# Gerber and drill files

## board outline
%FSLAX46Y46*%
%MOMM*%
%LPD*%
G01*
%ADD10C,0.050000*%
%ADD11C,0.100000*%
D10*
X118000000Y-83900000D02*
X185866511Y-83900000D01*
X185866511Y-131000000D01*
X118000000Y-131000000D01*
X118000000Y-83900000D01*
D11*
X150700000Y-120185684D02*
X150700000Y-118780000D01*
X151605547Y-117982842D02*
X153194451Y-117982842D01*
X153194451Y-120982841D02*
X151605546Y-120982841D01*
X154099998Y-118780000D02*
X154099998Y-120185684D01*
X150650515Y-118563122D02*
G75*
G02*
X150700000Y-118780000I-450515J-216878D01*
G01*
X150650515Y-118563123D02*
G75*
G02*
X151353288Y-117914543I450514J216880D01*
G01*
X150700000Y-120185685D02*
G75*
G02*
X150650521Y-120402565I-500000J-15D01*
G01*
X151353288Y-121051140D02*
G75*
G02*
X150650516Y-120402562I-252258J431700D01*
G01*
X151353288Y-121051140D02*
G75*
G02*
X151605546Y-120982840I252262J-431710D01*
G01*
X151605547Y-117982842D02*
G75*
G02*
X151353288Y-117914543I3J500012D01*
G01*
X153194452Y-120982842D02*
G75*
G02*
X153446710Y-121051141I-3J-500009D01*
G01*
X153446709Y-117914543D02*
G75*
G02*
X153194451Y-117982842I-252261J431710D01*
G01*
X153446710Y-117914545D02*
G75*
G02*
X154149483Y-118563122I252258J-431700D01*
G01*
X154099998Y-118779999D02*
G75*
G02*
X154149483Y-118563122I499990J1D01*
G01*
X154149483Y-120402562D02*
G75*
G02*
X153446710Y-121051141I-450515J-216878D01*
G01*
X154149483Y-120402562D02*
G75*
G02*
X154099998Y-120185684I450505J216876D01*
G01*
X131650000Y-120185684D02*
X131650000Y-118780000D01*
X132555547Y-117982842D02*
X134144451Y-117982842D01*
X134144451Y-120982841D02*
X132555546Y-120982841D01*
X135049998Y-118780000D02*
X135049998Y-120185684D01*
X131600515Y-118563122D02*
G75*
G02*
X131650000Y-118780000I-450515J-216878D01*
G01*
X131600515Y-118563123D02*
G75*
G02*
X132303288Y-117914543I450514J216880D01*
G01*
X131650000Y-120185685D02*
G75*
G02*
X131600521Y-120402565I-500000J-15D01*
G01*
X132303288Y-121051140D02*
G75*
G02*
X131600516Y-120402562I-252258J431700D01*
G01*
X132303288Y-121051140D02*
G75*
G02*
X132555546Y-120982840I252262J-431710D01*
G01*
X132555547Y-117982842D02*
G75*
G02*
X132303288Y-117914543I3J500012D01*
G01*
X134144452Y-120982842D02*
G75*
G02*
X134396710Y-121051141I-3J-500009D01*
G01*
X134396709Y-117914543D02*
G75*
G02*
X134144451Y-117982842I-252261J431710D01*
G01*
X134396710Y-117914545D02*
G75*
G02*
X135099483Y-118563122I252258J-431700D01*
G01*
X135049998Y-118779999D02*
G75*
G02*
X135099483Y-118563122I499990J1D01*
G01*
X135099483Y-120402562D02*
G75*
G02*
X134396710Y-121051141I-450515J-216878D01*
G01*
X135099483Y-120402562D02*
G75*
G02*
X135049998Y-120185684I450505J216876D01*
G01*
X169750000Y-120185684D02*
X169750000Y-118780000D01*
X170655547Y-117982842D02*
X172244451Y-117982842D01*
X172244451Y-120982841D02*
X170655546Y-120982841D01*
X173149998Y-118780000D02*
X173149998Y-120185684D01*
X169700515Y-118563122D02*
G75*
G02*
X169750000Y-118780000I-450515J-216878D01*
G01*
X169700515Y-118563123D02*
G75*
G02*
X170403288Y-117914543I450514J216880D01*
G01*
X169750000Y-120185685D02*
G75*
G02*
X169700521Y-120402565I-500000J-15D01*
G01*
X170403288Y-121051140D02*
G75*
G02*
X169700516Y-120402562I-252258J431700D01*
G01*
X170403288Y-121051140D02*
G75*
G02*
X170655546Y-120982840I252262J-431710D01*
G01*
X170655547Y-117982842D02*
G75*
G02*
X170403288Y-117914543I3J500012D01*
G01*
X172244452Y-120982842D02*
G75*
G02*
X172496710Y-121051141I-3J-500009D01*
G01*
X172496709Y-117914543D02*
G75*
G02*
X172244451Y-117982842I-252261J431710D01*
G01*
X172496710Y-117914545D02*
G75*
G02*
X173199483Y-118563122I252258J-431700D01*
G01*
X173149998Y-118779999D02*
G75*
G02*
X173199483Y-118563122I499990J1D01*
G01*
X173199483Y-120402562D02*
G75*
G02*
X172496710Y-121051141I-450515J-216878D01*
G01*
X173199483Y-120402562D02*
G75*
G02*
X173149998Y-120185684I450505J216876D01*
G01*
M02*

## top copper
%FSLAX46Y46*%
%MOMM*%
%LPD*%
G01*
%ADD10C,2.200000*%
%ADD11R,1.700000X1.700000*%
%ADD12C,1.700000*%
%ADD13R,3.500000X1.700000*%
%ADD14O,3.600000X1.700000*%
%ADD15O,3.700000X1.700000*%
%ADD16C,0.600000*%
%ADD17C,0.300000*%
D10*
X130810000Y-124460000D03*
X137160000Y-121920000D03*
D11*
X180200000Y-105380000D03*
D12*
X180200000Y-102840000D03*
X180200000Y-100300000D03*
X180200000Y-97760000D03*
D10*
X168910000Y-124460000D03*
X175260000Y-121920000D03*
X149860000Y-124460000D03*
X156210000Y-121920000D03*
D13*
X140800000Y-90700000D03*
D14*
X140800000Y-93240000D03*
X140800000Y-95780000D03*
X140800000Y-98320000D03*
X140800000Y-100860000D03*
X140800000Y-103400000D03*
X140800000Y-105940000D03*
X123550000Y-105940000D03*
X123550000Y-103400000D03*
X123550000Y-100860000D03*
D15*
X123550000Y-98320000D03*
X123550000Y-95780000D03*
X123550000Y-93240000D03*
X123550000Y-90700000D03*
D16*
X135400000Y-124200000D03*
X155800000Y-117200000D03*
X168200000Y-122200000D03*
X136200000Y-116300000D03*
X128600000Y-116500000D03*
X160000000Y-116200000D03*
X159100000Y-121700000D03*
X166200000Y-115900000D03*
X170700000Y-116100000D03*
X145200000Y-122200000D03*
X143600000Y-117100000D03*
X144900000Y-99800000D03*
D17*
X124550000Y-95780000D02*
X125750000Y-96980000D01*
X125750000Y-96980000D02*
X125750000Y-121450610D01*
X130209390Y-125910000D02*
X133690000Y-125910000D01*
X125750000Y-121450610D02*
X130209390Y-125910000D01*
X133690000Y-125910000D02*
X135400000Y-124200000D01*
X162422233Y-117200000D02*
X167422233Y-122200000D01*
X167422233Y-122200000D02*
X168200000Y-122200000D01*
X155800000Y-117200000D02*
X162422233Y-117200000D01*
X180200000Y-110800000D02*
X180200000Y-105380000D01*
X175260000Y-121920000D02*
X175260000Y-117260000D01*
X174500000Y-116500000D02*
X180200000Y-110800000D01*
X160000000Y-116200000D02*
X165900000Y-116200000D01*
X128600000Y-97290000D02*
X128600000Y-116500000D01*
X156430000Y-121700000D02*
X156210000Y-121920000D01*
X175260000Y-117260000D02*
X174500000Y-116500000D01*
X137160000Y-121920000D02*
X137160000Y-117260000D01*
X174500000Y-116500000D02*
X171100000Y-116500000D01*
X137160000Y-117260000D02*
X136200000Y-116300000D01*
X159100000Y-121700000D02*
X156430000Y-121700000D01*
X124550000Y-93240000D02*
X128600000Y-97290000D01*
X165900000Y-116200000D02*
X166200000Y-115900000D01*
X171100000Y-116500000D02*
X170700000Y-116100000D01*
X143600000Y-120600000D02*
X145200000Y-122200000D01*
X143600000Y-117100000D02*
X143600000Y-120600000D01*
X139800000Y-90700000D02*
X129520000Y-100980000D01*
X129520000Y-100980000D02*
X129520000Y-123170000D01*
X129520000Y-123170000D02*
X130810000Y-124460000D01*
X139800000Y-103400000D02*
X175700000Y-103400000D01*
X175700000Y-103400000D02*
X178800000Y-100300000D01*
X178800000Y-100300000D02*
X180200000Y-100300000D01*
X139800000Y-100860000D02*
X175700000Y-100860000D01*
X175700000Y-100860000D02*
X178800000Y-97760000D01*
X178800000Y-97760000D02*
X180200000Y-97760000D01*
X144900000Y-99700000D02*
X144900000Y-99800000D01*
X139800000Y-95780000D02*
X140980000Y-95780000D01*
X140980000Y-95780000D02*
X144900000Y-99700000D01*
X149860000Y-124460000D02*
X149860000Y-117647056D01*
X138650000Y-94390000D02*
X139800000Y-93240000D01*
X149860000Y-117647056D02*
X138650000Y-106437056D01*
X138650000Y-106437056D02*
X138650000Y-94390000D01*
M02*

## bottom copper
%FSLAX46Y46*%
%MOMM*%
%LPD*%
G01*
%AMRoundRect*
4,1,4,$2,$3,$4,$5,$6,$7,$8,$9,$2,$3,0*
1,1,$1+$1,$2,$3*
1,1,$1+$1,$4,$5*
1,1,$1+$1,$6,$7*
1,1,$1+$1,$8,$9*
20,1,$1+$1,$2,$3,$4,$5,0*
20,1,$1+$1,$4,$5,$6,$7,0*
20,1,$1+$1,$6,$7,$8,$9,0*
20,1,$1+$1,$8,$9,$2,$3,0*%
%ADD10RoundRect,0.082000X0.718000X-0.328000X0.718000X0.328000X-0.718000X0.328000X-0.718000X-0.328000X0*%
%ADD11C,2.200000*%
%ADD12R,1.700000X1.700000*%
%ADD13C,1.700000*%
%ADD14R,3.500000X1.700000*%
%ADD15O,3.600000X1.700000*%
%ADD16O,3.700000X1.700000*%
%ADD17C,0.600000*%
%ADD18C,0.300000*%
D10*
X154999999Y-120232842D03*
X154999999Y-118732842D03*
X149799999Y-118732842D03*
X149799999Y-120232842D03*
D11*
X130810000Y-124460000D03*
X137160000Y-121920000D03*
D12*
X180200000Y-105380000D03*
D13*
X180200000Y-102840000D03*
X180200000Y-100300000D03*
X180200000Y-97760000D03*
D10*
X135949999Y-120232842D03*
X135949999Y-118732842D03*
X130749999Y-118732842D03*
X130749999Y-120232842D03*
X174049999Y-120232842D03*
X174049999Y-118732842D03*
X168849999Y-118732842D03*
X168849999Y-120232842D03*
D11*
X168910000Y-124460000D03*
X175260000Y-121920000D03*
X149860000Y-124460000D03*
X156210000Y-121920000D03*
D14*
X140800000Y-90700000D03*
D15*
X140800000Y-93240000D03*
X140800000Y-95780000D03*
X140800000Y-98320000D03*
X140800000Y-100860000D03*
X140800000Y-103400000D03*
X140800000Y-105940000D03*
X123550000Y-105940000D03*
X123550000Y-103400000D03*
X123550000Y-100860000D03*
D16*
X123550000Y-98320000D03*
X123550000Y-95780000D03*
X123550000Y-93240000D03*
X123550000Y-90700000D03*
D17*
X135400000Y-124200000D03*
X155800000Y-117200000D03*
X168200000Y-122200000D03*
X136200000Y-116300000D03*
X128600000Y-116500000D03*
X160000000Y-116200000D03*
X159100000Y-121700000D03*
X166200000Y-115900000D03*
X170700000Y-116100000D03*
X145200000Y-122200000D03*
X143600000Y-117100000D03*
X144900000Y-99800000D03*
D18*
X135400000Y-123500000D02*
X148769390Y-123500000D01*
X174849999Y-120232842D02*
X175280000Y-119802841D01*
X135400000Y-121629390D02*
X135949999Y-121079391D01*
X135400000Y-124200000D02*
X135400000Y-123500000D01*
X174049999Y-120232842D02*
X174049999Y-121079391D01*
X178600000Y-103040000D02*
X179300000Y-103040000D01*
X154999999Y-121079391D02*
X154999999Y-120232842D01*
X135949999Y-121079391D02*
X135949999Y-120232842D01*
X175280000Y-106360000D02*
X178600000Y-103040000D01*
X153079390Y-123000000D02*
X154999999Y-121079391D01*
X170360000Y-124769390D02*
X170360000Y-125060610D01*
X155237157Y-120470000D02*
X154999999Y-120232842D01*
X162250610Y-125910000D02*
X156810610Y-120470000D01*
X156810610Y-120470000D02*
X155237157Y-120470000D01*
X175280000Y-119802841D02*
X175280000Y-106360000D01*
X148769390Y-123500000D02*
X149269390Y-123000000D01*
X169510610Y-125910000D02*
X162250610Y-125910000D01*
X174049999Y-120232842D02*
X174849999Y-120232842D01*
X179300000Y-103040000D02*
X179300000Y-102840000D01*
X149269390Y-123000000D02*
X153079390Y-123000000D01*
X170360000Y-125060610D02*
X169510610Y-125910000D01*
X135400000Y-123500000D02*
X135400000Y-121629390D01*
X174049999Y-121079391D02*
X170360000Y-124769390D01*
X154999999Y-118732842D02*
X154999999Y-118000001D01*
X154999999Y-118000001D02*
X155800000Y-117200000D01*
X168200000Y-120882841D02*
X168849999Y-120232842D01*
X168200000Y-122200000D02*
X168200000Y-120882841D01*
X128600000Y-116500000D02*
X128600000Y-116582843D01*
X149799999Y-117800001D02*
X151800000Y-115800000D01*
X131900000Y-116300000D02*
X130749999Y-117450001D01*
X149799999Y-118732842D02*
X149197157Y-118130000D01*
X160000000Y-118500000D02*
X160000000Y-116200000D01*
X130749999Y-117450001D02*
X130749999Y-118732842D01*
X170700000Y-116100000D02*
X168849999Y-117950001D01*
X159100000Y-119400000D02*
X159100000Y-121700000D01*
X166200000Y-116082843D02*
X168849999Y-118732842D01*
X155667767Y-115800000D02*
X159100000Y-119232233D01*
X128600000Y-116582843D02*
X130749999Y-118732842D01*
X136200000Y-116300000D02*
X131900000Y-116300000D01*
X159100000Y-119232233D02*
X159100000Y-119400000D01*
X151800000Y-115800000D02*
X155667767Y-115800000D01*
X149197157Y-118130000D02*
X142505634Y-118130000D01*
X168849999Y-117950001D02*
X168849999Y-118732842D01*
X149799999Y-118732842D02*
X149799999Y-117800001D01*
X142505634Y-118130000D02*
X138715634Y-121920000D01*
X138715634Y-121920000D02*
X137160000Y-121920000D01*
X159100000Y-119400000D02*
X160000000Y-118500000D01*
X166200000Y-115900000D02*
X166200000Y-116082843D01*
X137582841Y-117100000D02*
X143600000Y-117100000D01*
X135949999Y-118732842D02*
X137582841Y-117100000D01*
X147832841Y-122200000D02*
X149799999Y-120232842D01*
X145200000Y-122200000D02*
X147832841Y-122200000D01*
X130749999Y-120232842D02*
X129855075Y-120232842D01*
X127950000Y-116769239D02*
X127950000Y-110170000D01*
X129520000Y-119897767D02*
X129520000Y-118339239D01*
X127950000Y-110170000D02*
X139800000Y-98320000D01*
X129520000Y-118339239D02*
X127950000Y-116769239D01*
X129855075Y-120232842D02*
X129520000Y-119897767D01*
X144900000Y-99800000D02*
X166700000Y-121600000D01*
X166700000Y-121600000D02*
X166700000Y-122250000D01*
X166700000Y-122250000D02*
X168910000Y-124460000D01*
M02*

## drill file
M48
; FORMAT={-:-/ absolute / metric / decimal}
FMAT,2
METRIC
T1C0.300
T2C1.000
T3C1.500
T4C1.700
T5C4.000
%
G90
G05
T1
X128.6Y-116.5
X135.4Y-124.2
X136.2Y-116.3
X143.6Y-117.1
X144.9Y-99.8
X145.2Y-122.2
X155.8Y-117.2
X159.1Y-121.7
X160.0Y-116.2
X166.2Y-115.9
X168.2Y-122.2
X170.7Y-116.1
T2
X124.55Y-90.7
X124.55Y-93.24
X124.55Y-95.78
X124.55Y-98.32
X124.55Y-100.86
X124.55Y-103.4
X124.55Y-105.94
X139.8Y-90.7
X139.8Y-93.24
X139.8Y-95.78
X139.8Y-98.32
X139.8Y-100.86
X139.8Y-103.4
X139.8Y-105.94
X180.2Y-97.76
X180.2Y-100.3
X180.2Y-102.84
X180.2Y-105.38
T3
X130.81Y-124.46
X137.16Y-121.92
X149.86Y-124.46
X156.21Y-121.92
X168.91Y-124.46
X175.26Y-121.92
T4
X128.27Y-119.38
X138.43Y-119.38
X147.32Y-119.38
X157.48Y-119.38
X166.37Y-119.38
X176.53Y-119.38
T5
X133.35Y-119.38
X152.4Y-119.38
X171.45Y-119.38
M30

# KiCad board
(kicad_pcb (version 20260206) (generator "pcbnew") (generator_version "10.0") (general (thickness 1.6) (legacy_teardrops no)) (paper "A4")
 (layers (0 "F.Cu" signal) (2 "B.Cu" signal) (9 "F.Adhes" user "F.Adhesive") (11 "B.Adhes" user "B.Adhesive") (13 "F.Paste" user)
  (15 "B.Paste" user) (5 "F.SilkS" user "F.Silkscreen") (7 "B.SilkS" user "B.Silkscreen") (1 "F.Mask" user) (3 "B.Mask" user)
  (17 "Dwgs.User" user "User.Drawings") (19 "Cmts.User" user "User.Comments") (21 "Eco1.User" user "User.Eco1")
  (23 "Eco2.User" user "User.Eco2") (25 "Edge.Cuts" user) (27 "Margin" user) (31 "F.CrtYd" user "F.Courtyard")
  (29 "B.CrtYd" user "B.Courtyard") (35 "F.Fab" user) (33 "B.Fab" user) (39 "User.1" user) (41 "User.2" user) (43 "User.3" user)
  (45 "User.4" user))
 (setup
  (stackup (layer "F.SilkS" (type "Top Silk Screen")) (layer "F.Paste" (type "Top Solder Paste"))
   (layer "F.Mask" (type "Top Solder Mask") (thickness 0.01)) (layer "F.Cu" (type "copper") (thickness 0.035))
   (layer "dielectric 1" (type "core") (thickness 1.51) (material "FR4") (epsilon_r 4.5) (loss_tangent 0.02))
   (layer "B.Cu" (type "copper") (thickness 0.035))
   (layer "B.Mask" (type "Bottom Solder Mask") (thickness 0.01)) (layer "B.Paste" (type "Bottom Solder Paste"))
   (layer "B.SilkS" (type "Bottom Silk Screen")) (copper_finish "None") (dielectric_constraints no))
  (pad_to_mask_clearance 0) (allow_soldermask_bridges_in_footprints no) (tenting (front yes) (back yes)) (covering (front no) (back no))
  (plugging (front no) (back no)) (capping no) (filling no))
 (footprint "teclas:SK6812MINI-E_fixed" (layer "F.Cu") (at 152.4 119.38 180)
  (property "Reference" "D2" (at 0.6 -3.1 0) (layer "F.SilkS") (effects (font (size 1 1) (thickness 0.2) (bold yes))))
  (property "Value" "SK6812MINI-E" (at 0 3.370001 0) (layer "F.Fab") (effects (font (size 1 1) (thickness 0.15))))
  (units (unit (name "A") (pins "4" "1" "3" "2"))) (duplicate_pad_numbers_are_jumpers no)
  (fp_line (start 1.7 -0.805684) (end 1.7 0.6) (stroke (width 0.1) (type solid)) (layer "Edge.Cuts"))
  (fp_line (start 0.794453 1.397158) (end -0.794451 1.397158) (stroke (width 0.1) (type solid)) (layer "Edge.Cuts"))
  (fp_line (start -0.794451 -1.602841) (end 0.794454 -1.602841) (stroke (width 0.1) (type solid)) (layer "Edge.Cuts"))
  (fp_line (start -1.699998 0.6) (end -1.699998 -0.805684) (stroke (width 0.1) (type solid)) (layer "Edge.Cuts"))
  (fp_arc (start 1.749485 0.816878) (mid 1.712528 0.711226) (end 1.7 0.6) (stroke (width 0.1) (type solid)) (layer "Edge.Cuts"))
  (fp_arc (start 1.749485 0.816877) (mid 1.638073 1.401193) (end 1.046712 1.465457) (stroke (width 0.1) (type solid)) (layer "Edge.Cuts"))
  (fp_arc (start 1.7 -0.805685) (mid 1.712528 -0.91691) (end 1.749485 -1.022562) (stroke (width 0.1) (type solid)) (layer "Edge.Cuts"))
  (fp_arc (start 1.046712 -1.67114) (mid 1.638072 -1.606876) (end 1.749485 -1.022562) (stroke (width 0.1) (type solid)) (layer "Edge.Cuts"))
  (fp_arc (start 1.046712 -1.67114) (mid 0.925124 -1.620218) (end 0.794454 -1.602841) (stroke (width 0.1) (type solid)) (layer "Edge.Cuts"))
  (fp_arc (start 0.794453 1.397158) (mid 0.925124 1.414535) (end 1.046712 1.465457) (stroke (width 0.1) (type solid)) (layer "Edge.Cuts"))
  (fp_arc (start -0.794452 -1.602842) (mid -0.925122 -1.620219) (end -1.04671 -1.671141) (stroke (width 0.1) (type solid))
   (layer "Edge.Cuts"))
  (fp_arc (start -1.046709 1.465457) (mid -0.925121 1.414535) (end -0.794451 1.397158) (stroke (width 0.1) (type solid)) (layer "Edge.Cuts"))
  (fp_arc (start -1.04671 1.465455) (mid -1.638069 1.401192) (end -1.749483 0.816878) (stroke (width 0.1) (type solid)) (layer "Edge.Cuts"))
  (fp_arc (start -1.699998 0.600001) (mid -1.712526 0.711226) (end -1.749483 0.816878) (stroke (width 0.1) (type solid)) (layer "Edge.Cuts"))
  (fp_arc (start -1.749483 -1.022562) (mid -1.63807 -1.606877) (end -1.04671 -1.671141) (stroke (width 0.1) (type solid))
   (layer "Edge.Cuts"))
  (fp_arc (start -1.749483 -1.022562) (mid -1.712526 -0.91691) (end -1.699998 -0.805684) (stroke (width 0.1) (type solid))
   (layer "Edge.Cuts"))
  (pad "1" smd roundrect (at -2.599999 -0.852842 90) (size 0.82 1.6) (layers "B.Cu" "B.Mask" "B.Paste") (roundrect_rratio 0.1) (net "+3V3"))
  (pad "2" smd roundrect (at -2.599999 0.647158 90) (size 0.82 1.6) (layers "B.Cu" "B.Mask" "B.Paste") (roundrect_rratio 0.1)
   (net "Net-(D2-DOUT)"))
  (pad "3" smd roundrect (at 2.600001 0.647158 90) (size 0.82 1.6) (layers "B.Cu" "B.Mask" "B.Paste") (roundrect_rratio 0.1) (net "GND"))
  (pad "4" smd roundrect (at 2.600001 -0.852842 90) (size 0.82 1.6) (layers "B.Cu" "B.Mask" "B.Paste") (roundrect_rratio 0.1)
   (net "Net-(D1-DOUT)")))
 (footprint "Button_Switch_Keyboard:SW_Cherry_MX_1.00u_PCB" (layer "F.Cu") (at 130.81 124.46 180)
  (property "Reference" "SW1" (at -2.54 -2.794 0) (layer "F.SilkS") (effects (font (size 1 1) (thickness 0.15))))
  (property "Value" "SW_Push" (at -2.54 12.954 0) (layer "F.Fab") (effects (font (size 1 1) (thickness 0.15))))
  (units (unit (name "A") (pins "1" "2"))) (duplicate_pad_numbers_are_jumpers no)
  (pad "" np_thru_hole circle (at -7.62 5.08 180) (size 1.7 1.7) (drill 1.7) (layers "*.Cu" "*.Mask"))
  (pad "" np_thru_hole circle (at -2.54 5.08 180) (size 4 4) (drill 4) (layers "*.Cu" "*.Mask"))
  (pad "" np_thru_hole circle (at 2.54 5.08 180) (size 1.7 1.7) (drill 1.7) (layers "*.Cu" "*.Mask"))
  (pad "1" thru_hole circle (at 0 0 180) (size 2.2 2.2) (drill 1.5) (layers "*.Cu" "*.Mask") (remove_unused_layers no)
   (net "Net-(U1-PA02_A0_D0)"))
  (pad "2" thru_hole circle (at -6.35 2.54 180) (size 2.2 2.2) (drill 1.5) (layers "*.Cu" "*.Mask") (remove_unused_layers no) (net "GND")))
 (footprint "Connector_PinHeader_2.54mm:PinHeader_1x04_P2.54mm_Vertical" (layer "F.Cu") (at 180.2 105.38 180)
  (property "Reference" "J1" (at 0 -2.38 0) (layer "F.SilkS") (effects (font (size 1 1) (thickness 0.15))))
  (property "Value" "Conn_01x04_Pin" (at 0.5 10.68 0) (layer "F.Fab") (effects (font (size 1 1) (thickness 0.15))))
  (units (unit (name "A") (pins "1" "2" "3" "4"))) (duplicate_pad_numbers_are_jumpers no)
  (pad "1" thru_hole rect (at 0 0 180) (size 1.7 1.7) (drill 1) (layers "*.Cu" "*.Mask") (remove_unused_layers no) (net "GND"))
  (pad "2" thru_hole circle (at 0 2.54 180) (size 1.7 1.7) (drill 1) (layers "*.Cu" "*.Mask") (remove_unused_layers no) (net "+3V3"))
  (pad "3" thru_hole circle (at 0 5.08 180) (size 1.7 1.7) (drill 1) (layers "*.Cu" "*.Mask") (remove_unused_layers no)
   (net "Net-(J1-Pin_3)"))
  (pad "4" thru_hole circle (at 0 7.62 180) (size 1.7 1.7) (drill 1) (layers "*.Cu" "*.Mask") (remove_unused_layers no)
   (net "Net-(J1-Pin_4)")))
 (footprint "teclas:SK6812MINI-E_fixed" (layer "F.Cu") (at 133.35 119.38 180)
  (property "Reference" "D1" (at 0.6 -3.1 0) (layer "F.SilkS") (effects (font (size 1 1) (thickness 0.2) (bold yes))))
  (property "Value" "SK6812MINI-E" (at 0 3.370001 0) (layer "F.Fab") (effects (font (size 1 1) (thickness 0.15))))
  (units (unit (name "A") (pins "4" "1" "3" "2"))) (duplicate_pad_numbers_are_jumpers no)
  (fp_line (start 1.7 -0.805684) (end 1.7 0.6) (stroke (width 0.1) (type solid)) (layer "Edge.Cuts"))
  (fp_line (start 0.794453 1.397158) (end -0.794451 1.397158) (stroke (width 0.1) (type solid)) (layer "Edge.Cuts"))
  (fp_line (start -0.794451 -1.602841) (end 0.794454 -1.602841) (stroke (width 0.1) (type solid)) (layer "Edge.Cuts"))
  (fp_line (start -1.699998 0.6) (end -1.699998 -0.805684) (stroke (width 0.1) (type solid)) (layer "Edge.Cuts"))
  (fp_arc (start 1.749485 0.816878) (mid 1.712528 0.711226) (end 1.7 0.6) (stroke (width 0.1) (type solid)) (layer "Edge.Cuts"))
  (fp_arc (start 1.749485 0.816877) (mid 1.638073 1.401193) (end 1.046712 1.465457) (stroke (width 0.1) (type solid)) (layer "Edge.Cuts"))
  (fp_arc (start 1.7 -0.805685) (mid 1.712528 -0.91691) (end 1.749485 -1.022562) (stroke (width 0.1) (type solid)) (layer "Edge.Cuts"))
  (fp_arc (start 1.046712 -1.67114) (mid 1.638072 -1.606876) (end 1.749485 -1.022562) (stroke (width 0.1) (type solid)) (layer "Edge.Cuts"))
  (fp_arc (start 1.046712 -1.67114) (mid 0.925124 -1.620218) (end 0.794454 -1.602841) (stroke (width 0.1) (type solid)) (layer "Edge.Cuts"))
  (fp_arc (start 0.794453 1.397158) (mid 0.925124 1.414535) (end 1.046712 1.465457) (stroke (width 0.1) (type solid)) (layer "Edge.Cuts"))
  (fp_arc (start -0.794452 -1.602842) (mid -0.925122 -1.620219) (end -1.04671 -1.671141) (stroke (width 0.1) (type solid))
   (layer "Edge.Cuts"))
  (fp_arc (start -1.046709 1.465457) (mid -0.925121 1.414535) (end -0.794451 1.397158) (stroke (width 0.1) (type solid)) (layer "Edge.Cuts"))
  (fp_arc (start -1.04671 1.465455) (mid -1.638069 1.401192) (end -1.749483 0.816878) (stroke (width 0.1) (type solid)) (layer "Edge.Cuts"))
  (fp_arc (start -1.699998 0.600001) (mid -1.712526 0.711226) (end -1.749483 0.816878) (stroke (width 0.1) (type solid)) (layer "Edge.Cuts"))
  (fp_arc (start -1.749483 -1.022562) (mid -1.63807 -1.606877) (end -1.04671 -1.671141) (stroke (width 0.1) (type solid))
   (layer "Edge.Cuts"))
  (fp_arc (start -1.749483 -1.022562) (mid -1.712526 -0.91691) (end -1.699998 -0.805684) (stroke (width 0.1) (type solid))
   (layer "Edge.Cuts"))
  (pad "1" smd roundrect (at -2.599999 -0.852842 90) (size 0.82 1.6) (layers "B.Cu" "B.Mask" "B.Paste") (roundrect_rratio 0.1) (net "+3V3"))
  (pad "2" smd roundrect (at -2.599999 0.647158 90) (size 0.82 1.6) (layers "B.Cu" "B.Mask" "B.Paste") (roundrect_rratio 0.1)
   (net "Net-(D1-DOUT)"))
  (pad "3" smd roundrect (at 2.600001 0.647158 90) (size 0.82 1.6) (layers "B.Cu" "B.Mask" "B.Paste") (roundrect_rratio 0.1) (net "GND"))
  (pad "4" smd roundrect (at 2.600001 -0.852842 90) (size 0.82 1.6) (layers "B.Cu" "B.Mask" "B.Paste") (roundrect_rratio 0.1)
   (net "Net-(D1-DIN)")))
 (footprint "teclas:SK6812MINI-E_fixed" (layer "F.Cu") (at 171.45 119.38 180)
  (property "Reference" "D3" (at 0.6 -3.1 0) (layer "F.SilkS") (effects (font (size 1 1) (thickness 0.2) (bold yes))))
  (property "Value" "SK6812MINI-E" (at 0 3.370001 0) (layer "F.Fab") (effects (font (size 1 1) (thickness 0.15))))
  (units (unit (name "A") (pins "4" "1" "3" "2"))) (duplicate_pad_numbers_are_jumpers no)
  (fp_line (start 1.7 -0.805684) (end 1.7 0.6) (stroke (width 0.1) (type solid)) (layer "Edge.Cuts"))
  (fp_line (start 0.794453 1.397158) (end -0.794451 1.397158) (stroke (width 0.1) (type solid)) (layer "Edge.Cuts"))
  (fp_line (start -0.794451 -1.602841) (end 0.794454 -1.602841) (stroke (width 0.1) (type solid)) (layer "Edge.Cuts"))
  (fp_line (start -1.699998 0.6) (end -1.699998 -0.805684) (stroke (width 0.1) (type solid)) (layer "Edge.Cuts"))
  (fp_arc (start 1.749485 0.816878) (mid 1.712528 0.711226) (end 1.7 0.6) (stroke (width 0.1) (type solid)) (layer "Edge.Cuts"))
  (fp_arc (start 1.749485 0.816877) (mid 1.638073 1.401193) (end 1.046712 1.465457) (stroke (width 0.1) (type solid)) (layer "Edge.Cuts"))
  (fp_arc (start 1.7 -0.805685) (mid 1.712528 -0.91691) (end 1.749485 -1.022562) (stroke (width 0.1) (type solid)) (layer "Edge.Cuts"))
  (fp_arc (start 1.046712 -1.67114) (mid 1.638072 -1.606876) (end 1.749485 -1.022562) (stroke (width 0.1) (type solid)) (layer "Edge.Cuts"))
  (fp_arc (start 1.046712 -1.67114) (mid 0.925124 -1.620218) (end 0.794454 -1.602841) (stroke (width 0.1) (type solid)) (layer "Edge.Cuts"))
  (fp_arc (start 0.794453 1.397158) (mid 0.925124 1.414535) (end 1.046712 1.465457) (stroke (width 0.1) (type solid)) (layer "Edge.Cuts"))
  (fp_arc (start -0.794452 -1.602842) (mid -0.925122 -1.620219) (end -1.04671 -1.671141) (stroke (width 0.1) (type solid))
   (layer "Edge.Cuts"))
  (fp_arc (start -1.046709 1.465457) (mid -0.925121 1.414535) (end -0.794451 1.397158) (stroke (width 0.1) (type solid)) (layer "Edge.Cuts"))
  (fp_arc (start -1.04671 1.465455) (mid -1.638069 1.401192) (end -1.749483 0.816878) (stroke (width 0.1) (type solid)) (layer "Edge.Cuts"))
  (fp_arc (start -1.699998 0.600001) (mid -1.712526 0.711226) (end -1.749483 0.816878) (stroke (width 0.1) (type solid)) (layer "Edge.Cuts"))
  (fp_arc (start -1.749483 -1.022562) (mid -1.63807 -1.606877) (end -1.04671 -1.671141) (stroke (width 0.1) (type solid))
   (layer "Edge.Cuts"))
  (fp_arc (start -1.749483 -1.022562) (mid -1.712526 -0.91691) (end -1.699998 -0.805684) (stroke (width 0.1) (type solid))
   (layer "Edge.Cuts"))
  (pad "1" smd roundrect (at -2.599999 -0.852842 90) (size 0.82 1.6) (layers "B.Cu" "B.Mask" "B.Paste") (roundrect_rratio 0.1) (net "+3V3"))
  (pad "2" smd roundrect (at -2.599999 0.647158 90) (size 0.82 1.6) (layers "B.Cu" "B.Mask" "B.Paste") (roundrect_rratio 0.1)
   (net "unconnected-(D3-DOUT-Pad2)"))
  (pad "3" smd roundrect (at 2.600001 0.647158 90) (size 0.82 1.6) (layers "B.Cu" "B.Mask" "B.Paste") (roundrect_rratio 0.1) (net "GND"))
  (pad "4" smd roundrect (at 2.600001 -0.852842 90) (size 0.82 1.6) (layers "B.Cu" "B.Mask" "B.Paste") (roundrect_rratio 0.1)
   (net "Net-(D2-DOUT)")))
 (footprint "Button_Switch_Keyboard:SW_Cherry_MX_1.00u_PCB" (layer "F.Cu") (at 168.91 124.46 180)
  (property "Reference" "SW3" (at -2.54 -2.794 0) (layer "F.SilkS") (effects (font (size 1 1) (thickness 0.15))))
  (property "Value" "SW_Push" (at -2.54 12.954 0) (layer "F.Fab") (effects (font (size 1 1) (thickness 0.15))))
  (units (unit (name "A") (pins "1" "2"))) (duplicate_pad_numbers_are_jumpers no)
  (pad "" np_thru_hole circle (at -7.62 5.08 180) (size 1.7 1.7) (drill 1.7) (layers "*.Cu" "*.Mask"))
  (pad "" np_thru_hole circle (at -2.54 5.08 180) (size 4 4) (drill 4) (layers "*.Cu" "*.Mask"))
  (pad "" np_thru_hole circle (at 2.54 5.08 180) (size 1.7 1.7) (drill 1.7) (layers "*.Cu" "*.Mask"))
  (pad "1" thru_hole circle (at 0 0 180) (size 2.2 2.2) (drill 1.5) (layers "*.Cu" "*.Mask") (remove_unused_layers no)
   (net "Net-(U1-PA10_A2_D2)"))
  (pad "2" thru_hole circle (at -6.35 2.54 180) (size 2.2 2.2) (drill 1.5) (layers "*.Cu" "*.Mask") (remove_unused_layers no) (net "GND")))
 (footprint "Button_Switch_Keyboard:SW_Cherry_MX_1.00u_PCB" (layer "F.Cu") (at 149.86 124.46 180)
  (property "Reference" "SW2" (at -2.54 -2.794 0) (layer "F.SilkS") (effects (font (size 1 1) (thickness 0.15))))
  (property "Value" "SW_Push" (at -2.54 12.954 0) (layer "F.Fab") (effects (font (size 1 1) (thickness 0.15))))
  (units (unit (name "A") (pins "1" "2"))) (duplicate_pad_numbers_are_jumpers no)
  (pad "" np_thru_hole circle (at -7.62 5.08 180) (size 1.7 1.7) (drill 1.7) (layers "*.Cu" "*.Mask"))
  (pad "" np_thru_hole circle (at -2.54 5.08 180) (size 4 4) (drill 4) (layers "*.Cu" "*.Mask"))
  (pad "" np_thru_hole circle (at 2.54 5.08 180) (size 1.7 1.7) (drill 1.7) (layers "*.Cu" "*.Mask"))
  (pad "1" thru_hole circle (at 0 0 180) (size 2.2 2.2) (drill 1.5) (layers "*.Cu" "*.Mask") (remove_unused_layers no)
   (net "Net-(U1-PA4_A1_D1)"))
  (pad "2" thru_hole circle (at -6.35 2.54 180) (size 2.2 2.2) (drill 1.5) (layers "*.Cu" "*.Mask") (remove_unused_layers no) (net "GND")))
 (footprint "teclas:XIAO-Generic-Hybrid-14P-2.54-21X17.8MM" (layer "B.Cu") (at 132.175 98.32 180)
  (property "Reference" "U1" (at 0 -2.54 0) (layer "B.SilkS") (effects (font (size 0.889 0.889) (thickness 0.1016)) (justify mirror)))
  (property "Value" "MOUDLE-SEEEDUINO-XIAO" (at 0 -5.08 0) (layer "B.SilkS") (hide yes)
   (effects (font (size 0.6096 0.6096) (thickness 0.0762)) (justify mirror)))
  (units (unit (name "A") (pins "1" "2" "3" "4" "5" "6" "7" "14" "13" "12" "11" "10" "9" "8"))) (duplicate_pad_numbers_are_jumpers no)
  (pad "1" thru_hole rect (at -7.625 7.62 180) (size 3.5 1.7) (drill 1 (offset -1 0)) (layers "*.Cu" "*.Mask") (remove_unused_layers no)
   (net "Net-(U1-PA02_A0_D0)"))
  (pad "2" thru_hole oval (at -7.625 5.08 180) (size 3.6 1.7) (drill 1 (offset -1 0)) (layers "*.Cu" "*.Mask") (remove_unused_layers no)
   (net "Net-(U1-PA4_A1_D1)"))
  (pad "3" thru_hole oval (at -7.625 2.54 180) (size 3.6 1.7) (drill 1 (offset -1 0)) (layers "*.Cu" "*.Mask") (remove_unused_layers no)
   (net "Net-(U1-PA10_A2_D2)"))
  (pad "4" thru_hole oval (at -7.625 0 180) (size 3.6 1.7) (drill 1 (offset -1 0)) (layers "*.Cu" "*.Mask") (remove_unused_layers no)
   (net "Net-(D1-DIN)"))
  (pad "5" thru_hole oval (at -7.625 -2.54 180) (size 3.6 1.7) (drill 1 (offset -1 0)) (layers "*.Cu" "*.Mask") (remove_unused_layers no)
   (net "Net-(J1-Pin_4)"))
  (pad "6" thru_hole oval (at -7.625 -5.08) (size 3.6 1.7) (drill 1 (offset 1 0)) (layers "*.Cu" "*.Mask") (remove_unused_layers no)
   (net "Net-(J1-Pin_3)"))
  (pad "7" thru_hole oval (at -7.625 -7.62 180) (size 3.6 1.7) (drill 1 (offset -1 0)) (layers "*.Cu" "*.Mask") (remove_unused_layers no)
   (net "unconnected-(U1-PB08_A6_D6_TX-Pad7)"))
  (pad "8" thru_hole oval (at 7.625 -7.62 180) (size 3.6 1.7) (drill 1 (offset 1 0)) (layers "*.Cu" "*.Mask") (remove_unused_layers no)
   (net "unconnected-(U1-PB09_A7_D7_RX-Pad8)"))
  (pad "9" thru_hole oval (at 7.625 -5.08 180) (size 3.6 1.7) (drill 1 (offset 1 0)) (layers "*.Cu" "*.Mask") (remove_unused_layers no)
   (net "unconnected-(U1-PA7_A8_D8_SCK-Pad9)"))
  (pad "10" thru_hole oval (at 7.625 -2.54 180) (size 3.6 1.7) (drill 1 (offset 1 0)) (layers "*.Cu" "*.Mask") (remove_unused_layers no)
   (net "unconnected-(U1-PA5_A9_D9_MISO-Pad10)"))
  (pad "11" thru_hole oval (at 7.625 0 180) (size 3.7 1.7) (drill 1 (offset 1 0)) (layers "*.Cu" "*.Mask") (remove_unused_layers no)
   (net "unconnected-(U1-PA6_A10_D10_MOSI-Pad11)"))
  (pad "12" thru_hole oval (at 7.625 2.54 180) (size 3.7 1.7) (drill 1 (offset 1 0)) (layers "*.Cu" "*.Mask") (remove_unused_layers no)
   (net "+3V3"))
  (pad "13" thru_hole oval (at 7.625 5.08 180) (size 3.7 1.7) (drill 1 (offset 1 0)) (layers "*.Cu" "*.Mask") (remove_unused_layers no)
   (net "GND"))
  (pad "14" thru_hole oval (at 7.625 7.62 180) (size 3.7 1.7) (drill 1 (offset 1 0)) (layers "*.Cu" "*.Mask") (remove_unused_layers no)
   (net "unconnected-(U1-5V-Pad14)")))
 (gr_rect (start 118 83.9) (end 185.866511 131) (stroke (width 0.05) (type default)) (fill no) (layer "Edge.Cuts"))
 (segment (start 124.55 95.78) (end 125.75 96.98) (width 0.3) (layer "F.Cu") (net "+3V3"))
 (segment (start 125.75 96.98) (end 125.75 121.45061) (width 0.3) (layer "F.Cu") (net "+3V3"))
 (segment (start 130.20939 125.91) (end 133.69 125.91) (width 0.3) (layer "F.Cu") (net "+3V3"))
 (segment (start 125.75 121.45061) (end 130.20939 125.91) (width 0.3) (layer "F.Cu") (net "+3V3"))
 (segment (start 133.69 125.91) (end 135.4 124.2) (width 0.3) (layer "F.Cu") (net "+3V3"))
 (via (at 135.4 124.2) (size 0.6) (drill 0.3) (layers "F.Cu" "B.Cu") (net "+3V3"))
 (segment (start 135.4 123.5) (end 148.76939 123.5) (width 0.3) (layer "B.Cu") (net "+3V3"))
 (segment (start 174.849999 120.232842) (end 175.28 119.802841) (width 0.3) (layer "B.Cu") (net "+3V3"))
 (segment (start 135.4 121.62939) (end 135.949999 121.079391) (width 0.3) (layer "B.Cu") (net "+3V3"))
 (segment (start 135.4 124.2) (end 135.4 123.5) (width 0.3) (layer "B.Cu") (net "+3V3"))
 (segment (start 174.049999 120.232842) (end 174.049999 121.079391) (width 0.3) (layer "B.Cu") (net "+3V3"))
 (segment (start 178.6 103.04) (end 179.3 103.04) (width 0.3) (layer "B.Cu") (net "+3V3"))
 (segment (start 154.999999 121.079391) (end 154.999999 120.232842) (width 0.3) (layer "B.Cu") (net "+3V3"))
 (segment (start 135.949999 121.079391) (end 135.949999 120.232842) (width 0.3) (layer "B.Cu") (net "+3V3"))
 (segment (start 175.28 106.36) (end 178.6 103.04) (width 0.3) (layer "B.Cu") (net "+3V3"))
 (segment (start 153.07939 123) (end 154.999999 121.079391) (width 0.3) (layer "B.Cu") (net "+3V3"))
 (segment (start 170.36 124.76939) (end 170.36 125.06061) (width 0.3) (layer "B.Cu") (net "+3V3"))
 (segment (start 155.237157 120.47) (end 154.999999 120.232842) (width 0.3) (layer "B.Cu") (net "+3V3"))
 (segment (start 162.25061 125.91) (end 156.81061 120.47) (width 0.3) (layer "B.Cu") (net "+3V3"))
 (segment (start 156.81061 120.47) (end 155.237157 120.47) (width 0.3) (layer "B.Cu") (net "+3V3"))
 (segment (start 175.28 119.802841) (end 175.28 106.36) (width 0.3) (layer "B.Cu") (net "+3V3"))
 (segment (start 148.76939 123.5) (end 149.26939 123) (width 0.3) (layer "B.Cu") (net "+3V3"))
 (segment (start 169.51061 125.91) (end 162.25061 125.91) (width 0.3) (layer "B.Cu") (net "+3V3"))
 (segment (start 174.049999 120.232842) (end 174.849999 120.232842) (width 0.3) (layer "B.Cu") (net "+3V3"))
 (segment (start 179.3 103.04) (end 179.3 102.84) (width 0.3) (layer "B.Cu") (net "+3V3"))
 (segment (start 149.26939 123) (end 153.07939 123) (width 0.3) (layer "B.Cu") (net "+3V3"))
 (segment (start 170.36 125.06061) (end 169.51061 125.91) (width 0.3) (layer "B.Cu") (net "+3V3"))
 (segment (start 135.4 123.5) (end 135.4 121.62939) (width 0.3) (layer "B.Cu") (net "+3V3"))
 (segment (start 174.049999 121.079391) (end 170.36 124.76939) (width 0.3) (layer "B.Cu") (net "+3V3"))
 (segment (start 162.422233 117.2) (end 167.422233 122.2) (width 0.3) (layer "F.Cu") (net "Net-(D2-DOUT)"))
 (segment (start 167.422233 122.2) (end 168.2 122.2) (width 0.3) (layer "F.Cu") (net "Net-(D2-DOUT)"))
 (segment (start 155.8 117.2) (end 162.422233 117.2) (width 0.3) (layer "F.Cu") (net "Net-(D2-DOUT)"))
 (via (at 155.8 117.2) (size 0.6) (drill 0.3) (layers "F.Cu" "B.Cu") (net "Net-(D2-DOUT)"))
 (via (at 168.2 122.2) (size 0.6) (drill 0.3) (layers "F.Cu" "B.Cu") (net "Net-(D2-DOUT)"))
 (segment (start 154.999999 118.732842) (end 154.999999 118.000001) (width 0.3) (layer "B.Cu") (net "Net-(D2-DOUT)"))
 (segment (start 154.999999 118.000001) (end 155.8 117.2) (width 0.3) (layer "B.Cu") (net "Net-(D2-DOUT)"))
 (segment (start 168.2 120.882841) (end 168.849999 120.232842) (width 0.3) (layer "B.Cu") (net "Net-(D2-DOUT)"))
 (segment (start 168.2 122.2) (end 168.2 120.882841) (width 0.3) (layer "B.Cu") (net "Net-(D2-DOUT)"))
 (segment (start 180.2 110.8) (end 180.2 105.38) (width 0.3) (layer "F.Cu") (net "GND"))
 (segment (start 175.26 121.92) (end 175.26 117.26) (width 0.3) (layer "F.Cu") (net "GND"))
 (segment (start 174.5 116.5) (end 180.2 110.8) (width 0.3) (layer "F.Cu") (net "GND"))
 (segment (start 160 116.2) (end 165.9 116.2) (width 0.3) (layer "F.Cu") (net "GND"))
 (segment (start 128.6 97.29) (end 128.6 116.5) (width 0.3) (layer "F.Cu") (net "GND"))
 (segment (start 156.43 121.7) (end 156.21 121.92) (width 0.3) (layer "F.Cu") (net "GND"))
 (segment (start 175.26 117.26) (end 174.5 116.5) (width 0.3) (layer "F.Cu") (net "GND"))
 (segment (start 137.16 121.92) (end 137.16 117.26) (width 0.3) (layer "F.Cu") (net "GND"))
 (segment (start 174.5 116.5) (end 171.1 116.5) (width 0.3) (layer "F.Cu") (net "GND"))
 (segment (start 137.16 117.26) (end 136.2 116.3) (width 0.3) (layer "F.Cu") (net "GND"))
 (segment (start 159.1 121.7) (end 156.43 121.7) (width 0.3) (layer "F.Cu") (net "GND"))
 (segment (start 124.55 93.24) (end 128.6 97.29) (width 0.3) (layer "F.Cu") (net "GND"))
 (segment (start 165.9 116.2) (end 166.2 115.9) (width 0.3) (layer "F.Cu") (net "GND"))
 (segment (start 171.1 116.5) (end 170.7 116.1) (width 0.3) (layer "F.Cu") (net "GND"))
 (via (at 136.2 116.3) (size 0.6) (drill 0.3) (layers "F.Cu" "B.Cu") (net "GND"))
 (via (at 128.6 116.5) (size 0.6) (drill 0.3) (layers "F.Cu" "B.Cu") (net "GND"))
 (via (at 160 116.2) (size 0.6) (drill 0.3) (layers "F.Cu" "B.Cu") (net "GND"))
 (via (at 159.1 121.7) (size 0.6) (drill 0.3) (layers "F.Cu" "B.Cu") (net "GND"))
 (via (at 166.2 115.9) (size 0.6) (drill 0.3) (layers "F.Cu" "B.Cu") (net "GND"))
 (via (at 170.7 116.1) (size 0.6) (drill 0.3) (layers "F.Cu" "B.Cu") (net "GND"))
 (segment (start 128.6 116.5) (end 128.6 116.582843) (width 0.3) (layer "B.Cu") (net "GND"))
 (segment (start 149.799999 117.800001) (end 151.8 115.8) (width 0.3) (layer "B.Cu") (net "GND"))
 (segment (start 131.9 116.3) (end 130.749999 117.450001) (width 0.3) (layer "B.Cu") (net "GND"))
 (segment (start 149.799999 118.732842) (end 149.197157 118.13) (width 0.3) (layer "B.Cu") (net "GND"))
 (segment (start 160 118.5) (end 160 116.2) (width 0.3) (layer "B.Cu") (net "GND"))
 (segment (start 130.749999 117.450001) (end 130.749999 118.732842) (width 0.3) (layer "B.Cu") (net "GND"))
 (segment (start 170.7 116.1) (end 168.849999 117.950001) (width 0.3) (layer "B.Cu") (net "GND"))
 (segment (start 159.1 119.4) (end 159.1 121.7) (width 0.3) (layer "B.Cu") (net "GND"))
 (segment (start 166.2 116.082843) (end 168.849999 118.732842) (width 0.3) (layer "B.Cu") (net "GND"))
 (segment (start 155.667767 115.8) (end 159.1 119.232233) (width 0.3) (layer "B.Cu") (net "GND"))
 (segment (start 128.6 116.582843) (end 130.749999 118.732842) (width 0.3) (layer "B.Cu") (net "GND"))
 (segment (start 136.2 116.3) (end 131.9 116.3) (width 0.3) (layer "B.Cu") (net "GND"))
 (segment (start 159.1 119.232233) (end 159.1 119.4) (width 0.3) (layer "B.Cu") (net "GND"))
 (segment (start 151.8 115.8) (end 155.667767 115.8) (width 0.3) (layer "B.Cu") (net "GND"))
 (segment (start 149.197157 118.13) (end 142.505634 118.13) (width 0.3) (layer "B.Cu") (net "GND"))
 (segment (start 168.849999 117.950001) (end 168.849999 118.732842) (width 0.3) (layer "B.Cu") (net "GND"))
 (segment (start 149.799999 118.732842) (end 149.799999 117.800001) (width 0.3) (layer "B.Cu") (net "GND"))
 (segment (start 142.505634 118.13) (end 138.715634 121.92) (width 0.3) (layer "B.Cu") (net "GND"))
 (segment (start 138.715634 121.92) (end 137.16 121.92) (width 0.3) (layer "B.Cu") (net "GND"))
 (segment (start 159.1 119.4) (end 160 118.5) (width 0.3) (layer "B.Cu") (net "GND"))
 (segment (start 166.2 115.9) (end 166.2 116.082843) (width 0.3) (layer "B.Cu") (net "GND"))
 (segment (start 143.6 120.6) (end 145.2 122.2) (width 0.3) (layer "F.Cu") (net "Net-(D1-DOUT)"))
 (segment (start 143.6 117.1) (end 143.6 120.6) (width 0.3) (layer "F.Cu") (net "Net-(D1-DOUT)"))
 (via (at 145.2 122.2) (size 0.6) (drill 0.3) (layers "F.Cu" "B.Cu") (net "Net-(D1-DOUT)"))
 (via (at 143.6 117.1) (size 0.6) (drill 0.3) (layers "F.Cu" "B.Cu") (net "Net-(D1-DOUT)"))
 (segment (start 137.582841 117.1) (end 143.6 117.1) (width 0.3) (layer "B.Cu") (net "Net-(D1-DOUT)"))
 (segment (start 135.949999 118.732842) (end 137.582841 117.1) (width 0.3) (layer "B.Cu") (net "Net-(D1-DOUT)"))
 (segment (start 147.832841 122.2) (end 149.799999 120.232842) (width 0.3) (layer "B.Cu") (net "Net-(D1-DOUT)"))
 (segment (start 145.2 122.2) (end 147.832841 122.2) (width 0.3) (layer "B.Cu") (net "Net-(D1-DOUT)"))
 (segment (start 139.8 90.7) (end 129.52 100.98) (width 0.3) (layer "F.Cu") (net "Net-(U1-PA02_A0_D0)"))
 (segment (start 129.52 100.98) (end 129.52 123.17) (width 0.3) (layer "F.Cu") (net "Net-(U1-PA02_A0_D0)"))
 (segment (start 129.52 123.17) (end 130.81 124.46) (width 0.3) (layer "F.Cu") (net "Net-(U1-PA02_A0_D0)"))
 (segment (start 139.8 103.4) (end 175.7 103.4) (width 0.3) (layer "F.Cu") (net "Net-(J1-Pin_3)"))
 (segment (start 175.7 103.4) (end 178.8 100.3) (width 0.3) (layer "F.Cu") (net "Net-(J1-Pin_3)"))
 (segment (start 178.8 100.3) (end 180.2 100.3) (width 0.3) (layer "F.Cu") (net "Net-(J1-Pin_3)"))
 (segment (start 139.8 100.86) (end 175.7 100.86) (width 0.3) (layer "F.Cu") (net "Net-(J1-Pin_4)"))
 (segment (start 175.7 100.86) (end 178.8 97.76) (width 0.3) (layer "F.Cu") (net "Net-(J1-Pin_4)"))
 (segment (start 178.8 97.76) (end 180.2 97.76) (width 0.3) (layer "F.Cu") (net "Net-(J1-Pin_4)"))
 (segment (start 130.749999 120.232842) (end 129.855075 120.232842) (width 0.3) (layer "B.Cu") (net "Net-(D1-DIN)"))
 (segment (start 127.95 116.769239) (end 127.95 110.17) (width 0.3) (layer "B.Cu") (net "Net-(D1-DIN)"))
 (segment (start 129.52 119.897767) (end 129.52 118.339239) (width 0.3) (layer "B.Cu") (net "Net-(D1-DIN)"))
 (segment (start 127.95 110.17) (end 139.8 98.32) (width 0.3) (layer "B.Cu") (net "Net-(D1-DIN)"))
 (segment (start 129.52 118.339239) (end 127.95 116.769239) (width 0.3) (layer "B.Cu") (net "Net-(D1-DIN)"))
 (segment (start 129.855075 120.232842) (end 129.52 119.897767) (width 0.3) (layer "B.Cu") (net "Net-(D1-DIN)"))
 (segment (start 144.9 99.7) (end 144.9 99.8) (width 0.3) (layer "F.Cu") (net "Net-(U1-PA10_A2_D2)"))
 (segment (start 139.8 95.78) (end 140.98 95.78) (width 0.3) (layer "F.Cu") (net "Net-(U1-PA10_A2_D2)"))
 (segment (start 140.98 95.78) (end 144.9 99.7) (width 0.3) (layer "F.Cu") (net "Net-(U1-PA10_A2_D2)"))
 (via (at 144.9 99.8) (size 0.6) (drill 0.3) (layers "F.Cu" "B.Cu") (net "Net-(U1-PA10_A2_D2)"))
 (segment (start 144.9 99.8) (end 166.7 121.6) (width 0.3) (layer "B.Cu") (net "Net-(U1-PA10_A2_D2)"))
 (segment (start 166.7 121.6) (end 166.7 122.25) (width 0.3) (layer "B.Cu") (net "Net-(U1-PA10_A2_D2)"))
 (segment (start 166.7 122.25) (end 168.91 124.46) (width 0.3) (layer "B.Cu") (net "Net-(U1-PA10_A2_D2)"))
 (segment (start 149.86 124.46) (end 149.86 117.647056) (width 0.3) (layer "F.Cu") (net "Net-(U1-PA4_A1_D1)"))
 (segment (start 138.65 94.39) (end 139.8 93.24) (width 0.3) (layer "F.Cu") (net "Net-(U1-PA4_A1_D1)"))
 (segment (start 149.86 117.647056) (end 138.65 106.437056) (width 0.3) (layer "F.Cu") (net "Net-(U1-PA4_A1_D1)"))
 (segment (start 138.65 106.437056) (end 138.65 94.39) (width 0.3) (layer "F.Cu") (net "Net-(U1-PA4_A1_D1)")))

